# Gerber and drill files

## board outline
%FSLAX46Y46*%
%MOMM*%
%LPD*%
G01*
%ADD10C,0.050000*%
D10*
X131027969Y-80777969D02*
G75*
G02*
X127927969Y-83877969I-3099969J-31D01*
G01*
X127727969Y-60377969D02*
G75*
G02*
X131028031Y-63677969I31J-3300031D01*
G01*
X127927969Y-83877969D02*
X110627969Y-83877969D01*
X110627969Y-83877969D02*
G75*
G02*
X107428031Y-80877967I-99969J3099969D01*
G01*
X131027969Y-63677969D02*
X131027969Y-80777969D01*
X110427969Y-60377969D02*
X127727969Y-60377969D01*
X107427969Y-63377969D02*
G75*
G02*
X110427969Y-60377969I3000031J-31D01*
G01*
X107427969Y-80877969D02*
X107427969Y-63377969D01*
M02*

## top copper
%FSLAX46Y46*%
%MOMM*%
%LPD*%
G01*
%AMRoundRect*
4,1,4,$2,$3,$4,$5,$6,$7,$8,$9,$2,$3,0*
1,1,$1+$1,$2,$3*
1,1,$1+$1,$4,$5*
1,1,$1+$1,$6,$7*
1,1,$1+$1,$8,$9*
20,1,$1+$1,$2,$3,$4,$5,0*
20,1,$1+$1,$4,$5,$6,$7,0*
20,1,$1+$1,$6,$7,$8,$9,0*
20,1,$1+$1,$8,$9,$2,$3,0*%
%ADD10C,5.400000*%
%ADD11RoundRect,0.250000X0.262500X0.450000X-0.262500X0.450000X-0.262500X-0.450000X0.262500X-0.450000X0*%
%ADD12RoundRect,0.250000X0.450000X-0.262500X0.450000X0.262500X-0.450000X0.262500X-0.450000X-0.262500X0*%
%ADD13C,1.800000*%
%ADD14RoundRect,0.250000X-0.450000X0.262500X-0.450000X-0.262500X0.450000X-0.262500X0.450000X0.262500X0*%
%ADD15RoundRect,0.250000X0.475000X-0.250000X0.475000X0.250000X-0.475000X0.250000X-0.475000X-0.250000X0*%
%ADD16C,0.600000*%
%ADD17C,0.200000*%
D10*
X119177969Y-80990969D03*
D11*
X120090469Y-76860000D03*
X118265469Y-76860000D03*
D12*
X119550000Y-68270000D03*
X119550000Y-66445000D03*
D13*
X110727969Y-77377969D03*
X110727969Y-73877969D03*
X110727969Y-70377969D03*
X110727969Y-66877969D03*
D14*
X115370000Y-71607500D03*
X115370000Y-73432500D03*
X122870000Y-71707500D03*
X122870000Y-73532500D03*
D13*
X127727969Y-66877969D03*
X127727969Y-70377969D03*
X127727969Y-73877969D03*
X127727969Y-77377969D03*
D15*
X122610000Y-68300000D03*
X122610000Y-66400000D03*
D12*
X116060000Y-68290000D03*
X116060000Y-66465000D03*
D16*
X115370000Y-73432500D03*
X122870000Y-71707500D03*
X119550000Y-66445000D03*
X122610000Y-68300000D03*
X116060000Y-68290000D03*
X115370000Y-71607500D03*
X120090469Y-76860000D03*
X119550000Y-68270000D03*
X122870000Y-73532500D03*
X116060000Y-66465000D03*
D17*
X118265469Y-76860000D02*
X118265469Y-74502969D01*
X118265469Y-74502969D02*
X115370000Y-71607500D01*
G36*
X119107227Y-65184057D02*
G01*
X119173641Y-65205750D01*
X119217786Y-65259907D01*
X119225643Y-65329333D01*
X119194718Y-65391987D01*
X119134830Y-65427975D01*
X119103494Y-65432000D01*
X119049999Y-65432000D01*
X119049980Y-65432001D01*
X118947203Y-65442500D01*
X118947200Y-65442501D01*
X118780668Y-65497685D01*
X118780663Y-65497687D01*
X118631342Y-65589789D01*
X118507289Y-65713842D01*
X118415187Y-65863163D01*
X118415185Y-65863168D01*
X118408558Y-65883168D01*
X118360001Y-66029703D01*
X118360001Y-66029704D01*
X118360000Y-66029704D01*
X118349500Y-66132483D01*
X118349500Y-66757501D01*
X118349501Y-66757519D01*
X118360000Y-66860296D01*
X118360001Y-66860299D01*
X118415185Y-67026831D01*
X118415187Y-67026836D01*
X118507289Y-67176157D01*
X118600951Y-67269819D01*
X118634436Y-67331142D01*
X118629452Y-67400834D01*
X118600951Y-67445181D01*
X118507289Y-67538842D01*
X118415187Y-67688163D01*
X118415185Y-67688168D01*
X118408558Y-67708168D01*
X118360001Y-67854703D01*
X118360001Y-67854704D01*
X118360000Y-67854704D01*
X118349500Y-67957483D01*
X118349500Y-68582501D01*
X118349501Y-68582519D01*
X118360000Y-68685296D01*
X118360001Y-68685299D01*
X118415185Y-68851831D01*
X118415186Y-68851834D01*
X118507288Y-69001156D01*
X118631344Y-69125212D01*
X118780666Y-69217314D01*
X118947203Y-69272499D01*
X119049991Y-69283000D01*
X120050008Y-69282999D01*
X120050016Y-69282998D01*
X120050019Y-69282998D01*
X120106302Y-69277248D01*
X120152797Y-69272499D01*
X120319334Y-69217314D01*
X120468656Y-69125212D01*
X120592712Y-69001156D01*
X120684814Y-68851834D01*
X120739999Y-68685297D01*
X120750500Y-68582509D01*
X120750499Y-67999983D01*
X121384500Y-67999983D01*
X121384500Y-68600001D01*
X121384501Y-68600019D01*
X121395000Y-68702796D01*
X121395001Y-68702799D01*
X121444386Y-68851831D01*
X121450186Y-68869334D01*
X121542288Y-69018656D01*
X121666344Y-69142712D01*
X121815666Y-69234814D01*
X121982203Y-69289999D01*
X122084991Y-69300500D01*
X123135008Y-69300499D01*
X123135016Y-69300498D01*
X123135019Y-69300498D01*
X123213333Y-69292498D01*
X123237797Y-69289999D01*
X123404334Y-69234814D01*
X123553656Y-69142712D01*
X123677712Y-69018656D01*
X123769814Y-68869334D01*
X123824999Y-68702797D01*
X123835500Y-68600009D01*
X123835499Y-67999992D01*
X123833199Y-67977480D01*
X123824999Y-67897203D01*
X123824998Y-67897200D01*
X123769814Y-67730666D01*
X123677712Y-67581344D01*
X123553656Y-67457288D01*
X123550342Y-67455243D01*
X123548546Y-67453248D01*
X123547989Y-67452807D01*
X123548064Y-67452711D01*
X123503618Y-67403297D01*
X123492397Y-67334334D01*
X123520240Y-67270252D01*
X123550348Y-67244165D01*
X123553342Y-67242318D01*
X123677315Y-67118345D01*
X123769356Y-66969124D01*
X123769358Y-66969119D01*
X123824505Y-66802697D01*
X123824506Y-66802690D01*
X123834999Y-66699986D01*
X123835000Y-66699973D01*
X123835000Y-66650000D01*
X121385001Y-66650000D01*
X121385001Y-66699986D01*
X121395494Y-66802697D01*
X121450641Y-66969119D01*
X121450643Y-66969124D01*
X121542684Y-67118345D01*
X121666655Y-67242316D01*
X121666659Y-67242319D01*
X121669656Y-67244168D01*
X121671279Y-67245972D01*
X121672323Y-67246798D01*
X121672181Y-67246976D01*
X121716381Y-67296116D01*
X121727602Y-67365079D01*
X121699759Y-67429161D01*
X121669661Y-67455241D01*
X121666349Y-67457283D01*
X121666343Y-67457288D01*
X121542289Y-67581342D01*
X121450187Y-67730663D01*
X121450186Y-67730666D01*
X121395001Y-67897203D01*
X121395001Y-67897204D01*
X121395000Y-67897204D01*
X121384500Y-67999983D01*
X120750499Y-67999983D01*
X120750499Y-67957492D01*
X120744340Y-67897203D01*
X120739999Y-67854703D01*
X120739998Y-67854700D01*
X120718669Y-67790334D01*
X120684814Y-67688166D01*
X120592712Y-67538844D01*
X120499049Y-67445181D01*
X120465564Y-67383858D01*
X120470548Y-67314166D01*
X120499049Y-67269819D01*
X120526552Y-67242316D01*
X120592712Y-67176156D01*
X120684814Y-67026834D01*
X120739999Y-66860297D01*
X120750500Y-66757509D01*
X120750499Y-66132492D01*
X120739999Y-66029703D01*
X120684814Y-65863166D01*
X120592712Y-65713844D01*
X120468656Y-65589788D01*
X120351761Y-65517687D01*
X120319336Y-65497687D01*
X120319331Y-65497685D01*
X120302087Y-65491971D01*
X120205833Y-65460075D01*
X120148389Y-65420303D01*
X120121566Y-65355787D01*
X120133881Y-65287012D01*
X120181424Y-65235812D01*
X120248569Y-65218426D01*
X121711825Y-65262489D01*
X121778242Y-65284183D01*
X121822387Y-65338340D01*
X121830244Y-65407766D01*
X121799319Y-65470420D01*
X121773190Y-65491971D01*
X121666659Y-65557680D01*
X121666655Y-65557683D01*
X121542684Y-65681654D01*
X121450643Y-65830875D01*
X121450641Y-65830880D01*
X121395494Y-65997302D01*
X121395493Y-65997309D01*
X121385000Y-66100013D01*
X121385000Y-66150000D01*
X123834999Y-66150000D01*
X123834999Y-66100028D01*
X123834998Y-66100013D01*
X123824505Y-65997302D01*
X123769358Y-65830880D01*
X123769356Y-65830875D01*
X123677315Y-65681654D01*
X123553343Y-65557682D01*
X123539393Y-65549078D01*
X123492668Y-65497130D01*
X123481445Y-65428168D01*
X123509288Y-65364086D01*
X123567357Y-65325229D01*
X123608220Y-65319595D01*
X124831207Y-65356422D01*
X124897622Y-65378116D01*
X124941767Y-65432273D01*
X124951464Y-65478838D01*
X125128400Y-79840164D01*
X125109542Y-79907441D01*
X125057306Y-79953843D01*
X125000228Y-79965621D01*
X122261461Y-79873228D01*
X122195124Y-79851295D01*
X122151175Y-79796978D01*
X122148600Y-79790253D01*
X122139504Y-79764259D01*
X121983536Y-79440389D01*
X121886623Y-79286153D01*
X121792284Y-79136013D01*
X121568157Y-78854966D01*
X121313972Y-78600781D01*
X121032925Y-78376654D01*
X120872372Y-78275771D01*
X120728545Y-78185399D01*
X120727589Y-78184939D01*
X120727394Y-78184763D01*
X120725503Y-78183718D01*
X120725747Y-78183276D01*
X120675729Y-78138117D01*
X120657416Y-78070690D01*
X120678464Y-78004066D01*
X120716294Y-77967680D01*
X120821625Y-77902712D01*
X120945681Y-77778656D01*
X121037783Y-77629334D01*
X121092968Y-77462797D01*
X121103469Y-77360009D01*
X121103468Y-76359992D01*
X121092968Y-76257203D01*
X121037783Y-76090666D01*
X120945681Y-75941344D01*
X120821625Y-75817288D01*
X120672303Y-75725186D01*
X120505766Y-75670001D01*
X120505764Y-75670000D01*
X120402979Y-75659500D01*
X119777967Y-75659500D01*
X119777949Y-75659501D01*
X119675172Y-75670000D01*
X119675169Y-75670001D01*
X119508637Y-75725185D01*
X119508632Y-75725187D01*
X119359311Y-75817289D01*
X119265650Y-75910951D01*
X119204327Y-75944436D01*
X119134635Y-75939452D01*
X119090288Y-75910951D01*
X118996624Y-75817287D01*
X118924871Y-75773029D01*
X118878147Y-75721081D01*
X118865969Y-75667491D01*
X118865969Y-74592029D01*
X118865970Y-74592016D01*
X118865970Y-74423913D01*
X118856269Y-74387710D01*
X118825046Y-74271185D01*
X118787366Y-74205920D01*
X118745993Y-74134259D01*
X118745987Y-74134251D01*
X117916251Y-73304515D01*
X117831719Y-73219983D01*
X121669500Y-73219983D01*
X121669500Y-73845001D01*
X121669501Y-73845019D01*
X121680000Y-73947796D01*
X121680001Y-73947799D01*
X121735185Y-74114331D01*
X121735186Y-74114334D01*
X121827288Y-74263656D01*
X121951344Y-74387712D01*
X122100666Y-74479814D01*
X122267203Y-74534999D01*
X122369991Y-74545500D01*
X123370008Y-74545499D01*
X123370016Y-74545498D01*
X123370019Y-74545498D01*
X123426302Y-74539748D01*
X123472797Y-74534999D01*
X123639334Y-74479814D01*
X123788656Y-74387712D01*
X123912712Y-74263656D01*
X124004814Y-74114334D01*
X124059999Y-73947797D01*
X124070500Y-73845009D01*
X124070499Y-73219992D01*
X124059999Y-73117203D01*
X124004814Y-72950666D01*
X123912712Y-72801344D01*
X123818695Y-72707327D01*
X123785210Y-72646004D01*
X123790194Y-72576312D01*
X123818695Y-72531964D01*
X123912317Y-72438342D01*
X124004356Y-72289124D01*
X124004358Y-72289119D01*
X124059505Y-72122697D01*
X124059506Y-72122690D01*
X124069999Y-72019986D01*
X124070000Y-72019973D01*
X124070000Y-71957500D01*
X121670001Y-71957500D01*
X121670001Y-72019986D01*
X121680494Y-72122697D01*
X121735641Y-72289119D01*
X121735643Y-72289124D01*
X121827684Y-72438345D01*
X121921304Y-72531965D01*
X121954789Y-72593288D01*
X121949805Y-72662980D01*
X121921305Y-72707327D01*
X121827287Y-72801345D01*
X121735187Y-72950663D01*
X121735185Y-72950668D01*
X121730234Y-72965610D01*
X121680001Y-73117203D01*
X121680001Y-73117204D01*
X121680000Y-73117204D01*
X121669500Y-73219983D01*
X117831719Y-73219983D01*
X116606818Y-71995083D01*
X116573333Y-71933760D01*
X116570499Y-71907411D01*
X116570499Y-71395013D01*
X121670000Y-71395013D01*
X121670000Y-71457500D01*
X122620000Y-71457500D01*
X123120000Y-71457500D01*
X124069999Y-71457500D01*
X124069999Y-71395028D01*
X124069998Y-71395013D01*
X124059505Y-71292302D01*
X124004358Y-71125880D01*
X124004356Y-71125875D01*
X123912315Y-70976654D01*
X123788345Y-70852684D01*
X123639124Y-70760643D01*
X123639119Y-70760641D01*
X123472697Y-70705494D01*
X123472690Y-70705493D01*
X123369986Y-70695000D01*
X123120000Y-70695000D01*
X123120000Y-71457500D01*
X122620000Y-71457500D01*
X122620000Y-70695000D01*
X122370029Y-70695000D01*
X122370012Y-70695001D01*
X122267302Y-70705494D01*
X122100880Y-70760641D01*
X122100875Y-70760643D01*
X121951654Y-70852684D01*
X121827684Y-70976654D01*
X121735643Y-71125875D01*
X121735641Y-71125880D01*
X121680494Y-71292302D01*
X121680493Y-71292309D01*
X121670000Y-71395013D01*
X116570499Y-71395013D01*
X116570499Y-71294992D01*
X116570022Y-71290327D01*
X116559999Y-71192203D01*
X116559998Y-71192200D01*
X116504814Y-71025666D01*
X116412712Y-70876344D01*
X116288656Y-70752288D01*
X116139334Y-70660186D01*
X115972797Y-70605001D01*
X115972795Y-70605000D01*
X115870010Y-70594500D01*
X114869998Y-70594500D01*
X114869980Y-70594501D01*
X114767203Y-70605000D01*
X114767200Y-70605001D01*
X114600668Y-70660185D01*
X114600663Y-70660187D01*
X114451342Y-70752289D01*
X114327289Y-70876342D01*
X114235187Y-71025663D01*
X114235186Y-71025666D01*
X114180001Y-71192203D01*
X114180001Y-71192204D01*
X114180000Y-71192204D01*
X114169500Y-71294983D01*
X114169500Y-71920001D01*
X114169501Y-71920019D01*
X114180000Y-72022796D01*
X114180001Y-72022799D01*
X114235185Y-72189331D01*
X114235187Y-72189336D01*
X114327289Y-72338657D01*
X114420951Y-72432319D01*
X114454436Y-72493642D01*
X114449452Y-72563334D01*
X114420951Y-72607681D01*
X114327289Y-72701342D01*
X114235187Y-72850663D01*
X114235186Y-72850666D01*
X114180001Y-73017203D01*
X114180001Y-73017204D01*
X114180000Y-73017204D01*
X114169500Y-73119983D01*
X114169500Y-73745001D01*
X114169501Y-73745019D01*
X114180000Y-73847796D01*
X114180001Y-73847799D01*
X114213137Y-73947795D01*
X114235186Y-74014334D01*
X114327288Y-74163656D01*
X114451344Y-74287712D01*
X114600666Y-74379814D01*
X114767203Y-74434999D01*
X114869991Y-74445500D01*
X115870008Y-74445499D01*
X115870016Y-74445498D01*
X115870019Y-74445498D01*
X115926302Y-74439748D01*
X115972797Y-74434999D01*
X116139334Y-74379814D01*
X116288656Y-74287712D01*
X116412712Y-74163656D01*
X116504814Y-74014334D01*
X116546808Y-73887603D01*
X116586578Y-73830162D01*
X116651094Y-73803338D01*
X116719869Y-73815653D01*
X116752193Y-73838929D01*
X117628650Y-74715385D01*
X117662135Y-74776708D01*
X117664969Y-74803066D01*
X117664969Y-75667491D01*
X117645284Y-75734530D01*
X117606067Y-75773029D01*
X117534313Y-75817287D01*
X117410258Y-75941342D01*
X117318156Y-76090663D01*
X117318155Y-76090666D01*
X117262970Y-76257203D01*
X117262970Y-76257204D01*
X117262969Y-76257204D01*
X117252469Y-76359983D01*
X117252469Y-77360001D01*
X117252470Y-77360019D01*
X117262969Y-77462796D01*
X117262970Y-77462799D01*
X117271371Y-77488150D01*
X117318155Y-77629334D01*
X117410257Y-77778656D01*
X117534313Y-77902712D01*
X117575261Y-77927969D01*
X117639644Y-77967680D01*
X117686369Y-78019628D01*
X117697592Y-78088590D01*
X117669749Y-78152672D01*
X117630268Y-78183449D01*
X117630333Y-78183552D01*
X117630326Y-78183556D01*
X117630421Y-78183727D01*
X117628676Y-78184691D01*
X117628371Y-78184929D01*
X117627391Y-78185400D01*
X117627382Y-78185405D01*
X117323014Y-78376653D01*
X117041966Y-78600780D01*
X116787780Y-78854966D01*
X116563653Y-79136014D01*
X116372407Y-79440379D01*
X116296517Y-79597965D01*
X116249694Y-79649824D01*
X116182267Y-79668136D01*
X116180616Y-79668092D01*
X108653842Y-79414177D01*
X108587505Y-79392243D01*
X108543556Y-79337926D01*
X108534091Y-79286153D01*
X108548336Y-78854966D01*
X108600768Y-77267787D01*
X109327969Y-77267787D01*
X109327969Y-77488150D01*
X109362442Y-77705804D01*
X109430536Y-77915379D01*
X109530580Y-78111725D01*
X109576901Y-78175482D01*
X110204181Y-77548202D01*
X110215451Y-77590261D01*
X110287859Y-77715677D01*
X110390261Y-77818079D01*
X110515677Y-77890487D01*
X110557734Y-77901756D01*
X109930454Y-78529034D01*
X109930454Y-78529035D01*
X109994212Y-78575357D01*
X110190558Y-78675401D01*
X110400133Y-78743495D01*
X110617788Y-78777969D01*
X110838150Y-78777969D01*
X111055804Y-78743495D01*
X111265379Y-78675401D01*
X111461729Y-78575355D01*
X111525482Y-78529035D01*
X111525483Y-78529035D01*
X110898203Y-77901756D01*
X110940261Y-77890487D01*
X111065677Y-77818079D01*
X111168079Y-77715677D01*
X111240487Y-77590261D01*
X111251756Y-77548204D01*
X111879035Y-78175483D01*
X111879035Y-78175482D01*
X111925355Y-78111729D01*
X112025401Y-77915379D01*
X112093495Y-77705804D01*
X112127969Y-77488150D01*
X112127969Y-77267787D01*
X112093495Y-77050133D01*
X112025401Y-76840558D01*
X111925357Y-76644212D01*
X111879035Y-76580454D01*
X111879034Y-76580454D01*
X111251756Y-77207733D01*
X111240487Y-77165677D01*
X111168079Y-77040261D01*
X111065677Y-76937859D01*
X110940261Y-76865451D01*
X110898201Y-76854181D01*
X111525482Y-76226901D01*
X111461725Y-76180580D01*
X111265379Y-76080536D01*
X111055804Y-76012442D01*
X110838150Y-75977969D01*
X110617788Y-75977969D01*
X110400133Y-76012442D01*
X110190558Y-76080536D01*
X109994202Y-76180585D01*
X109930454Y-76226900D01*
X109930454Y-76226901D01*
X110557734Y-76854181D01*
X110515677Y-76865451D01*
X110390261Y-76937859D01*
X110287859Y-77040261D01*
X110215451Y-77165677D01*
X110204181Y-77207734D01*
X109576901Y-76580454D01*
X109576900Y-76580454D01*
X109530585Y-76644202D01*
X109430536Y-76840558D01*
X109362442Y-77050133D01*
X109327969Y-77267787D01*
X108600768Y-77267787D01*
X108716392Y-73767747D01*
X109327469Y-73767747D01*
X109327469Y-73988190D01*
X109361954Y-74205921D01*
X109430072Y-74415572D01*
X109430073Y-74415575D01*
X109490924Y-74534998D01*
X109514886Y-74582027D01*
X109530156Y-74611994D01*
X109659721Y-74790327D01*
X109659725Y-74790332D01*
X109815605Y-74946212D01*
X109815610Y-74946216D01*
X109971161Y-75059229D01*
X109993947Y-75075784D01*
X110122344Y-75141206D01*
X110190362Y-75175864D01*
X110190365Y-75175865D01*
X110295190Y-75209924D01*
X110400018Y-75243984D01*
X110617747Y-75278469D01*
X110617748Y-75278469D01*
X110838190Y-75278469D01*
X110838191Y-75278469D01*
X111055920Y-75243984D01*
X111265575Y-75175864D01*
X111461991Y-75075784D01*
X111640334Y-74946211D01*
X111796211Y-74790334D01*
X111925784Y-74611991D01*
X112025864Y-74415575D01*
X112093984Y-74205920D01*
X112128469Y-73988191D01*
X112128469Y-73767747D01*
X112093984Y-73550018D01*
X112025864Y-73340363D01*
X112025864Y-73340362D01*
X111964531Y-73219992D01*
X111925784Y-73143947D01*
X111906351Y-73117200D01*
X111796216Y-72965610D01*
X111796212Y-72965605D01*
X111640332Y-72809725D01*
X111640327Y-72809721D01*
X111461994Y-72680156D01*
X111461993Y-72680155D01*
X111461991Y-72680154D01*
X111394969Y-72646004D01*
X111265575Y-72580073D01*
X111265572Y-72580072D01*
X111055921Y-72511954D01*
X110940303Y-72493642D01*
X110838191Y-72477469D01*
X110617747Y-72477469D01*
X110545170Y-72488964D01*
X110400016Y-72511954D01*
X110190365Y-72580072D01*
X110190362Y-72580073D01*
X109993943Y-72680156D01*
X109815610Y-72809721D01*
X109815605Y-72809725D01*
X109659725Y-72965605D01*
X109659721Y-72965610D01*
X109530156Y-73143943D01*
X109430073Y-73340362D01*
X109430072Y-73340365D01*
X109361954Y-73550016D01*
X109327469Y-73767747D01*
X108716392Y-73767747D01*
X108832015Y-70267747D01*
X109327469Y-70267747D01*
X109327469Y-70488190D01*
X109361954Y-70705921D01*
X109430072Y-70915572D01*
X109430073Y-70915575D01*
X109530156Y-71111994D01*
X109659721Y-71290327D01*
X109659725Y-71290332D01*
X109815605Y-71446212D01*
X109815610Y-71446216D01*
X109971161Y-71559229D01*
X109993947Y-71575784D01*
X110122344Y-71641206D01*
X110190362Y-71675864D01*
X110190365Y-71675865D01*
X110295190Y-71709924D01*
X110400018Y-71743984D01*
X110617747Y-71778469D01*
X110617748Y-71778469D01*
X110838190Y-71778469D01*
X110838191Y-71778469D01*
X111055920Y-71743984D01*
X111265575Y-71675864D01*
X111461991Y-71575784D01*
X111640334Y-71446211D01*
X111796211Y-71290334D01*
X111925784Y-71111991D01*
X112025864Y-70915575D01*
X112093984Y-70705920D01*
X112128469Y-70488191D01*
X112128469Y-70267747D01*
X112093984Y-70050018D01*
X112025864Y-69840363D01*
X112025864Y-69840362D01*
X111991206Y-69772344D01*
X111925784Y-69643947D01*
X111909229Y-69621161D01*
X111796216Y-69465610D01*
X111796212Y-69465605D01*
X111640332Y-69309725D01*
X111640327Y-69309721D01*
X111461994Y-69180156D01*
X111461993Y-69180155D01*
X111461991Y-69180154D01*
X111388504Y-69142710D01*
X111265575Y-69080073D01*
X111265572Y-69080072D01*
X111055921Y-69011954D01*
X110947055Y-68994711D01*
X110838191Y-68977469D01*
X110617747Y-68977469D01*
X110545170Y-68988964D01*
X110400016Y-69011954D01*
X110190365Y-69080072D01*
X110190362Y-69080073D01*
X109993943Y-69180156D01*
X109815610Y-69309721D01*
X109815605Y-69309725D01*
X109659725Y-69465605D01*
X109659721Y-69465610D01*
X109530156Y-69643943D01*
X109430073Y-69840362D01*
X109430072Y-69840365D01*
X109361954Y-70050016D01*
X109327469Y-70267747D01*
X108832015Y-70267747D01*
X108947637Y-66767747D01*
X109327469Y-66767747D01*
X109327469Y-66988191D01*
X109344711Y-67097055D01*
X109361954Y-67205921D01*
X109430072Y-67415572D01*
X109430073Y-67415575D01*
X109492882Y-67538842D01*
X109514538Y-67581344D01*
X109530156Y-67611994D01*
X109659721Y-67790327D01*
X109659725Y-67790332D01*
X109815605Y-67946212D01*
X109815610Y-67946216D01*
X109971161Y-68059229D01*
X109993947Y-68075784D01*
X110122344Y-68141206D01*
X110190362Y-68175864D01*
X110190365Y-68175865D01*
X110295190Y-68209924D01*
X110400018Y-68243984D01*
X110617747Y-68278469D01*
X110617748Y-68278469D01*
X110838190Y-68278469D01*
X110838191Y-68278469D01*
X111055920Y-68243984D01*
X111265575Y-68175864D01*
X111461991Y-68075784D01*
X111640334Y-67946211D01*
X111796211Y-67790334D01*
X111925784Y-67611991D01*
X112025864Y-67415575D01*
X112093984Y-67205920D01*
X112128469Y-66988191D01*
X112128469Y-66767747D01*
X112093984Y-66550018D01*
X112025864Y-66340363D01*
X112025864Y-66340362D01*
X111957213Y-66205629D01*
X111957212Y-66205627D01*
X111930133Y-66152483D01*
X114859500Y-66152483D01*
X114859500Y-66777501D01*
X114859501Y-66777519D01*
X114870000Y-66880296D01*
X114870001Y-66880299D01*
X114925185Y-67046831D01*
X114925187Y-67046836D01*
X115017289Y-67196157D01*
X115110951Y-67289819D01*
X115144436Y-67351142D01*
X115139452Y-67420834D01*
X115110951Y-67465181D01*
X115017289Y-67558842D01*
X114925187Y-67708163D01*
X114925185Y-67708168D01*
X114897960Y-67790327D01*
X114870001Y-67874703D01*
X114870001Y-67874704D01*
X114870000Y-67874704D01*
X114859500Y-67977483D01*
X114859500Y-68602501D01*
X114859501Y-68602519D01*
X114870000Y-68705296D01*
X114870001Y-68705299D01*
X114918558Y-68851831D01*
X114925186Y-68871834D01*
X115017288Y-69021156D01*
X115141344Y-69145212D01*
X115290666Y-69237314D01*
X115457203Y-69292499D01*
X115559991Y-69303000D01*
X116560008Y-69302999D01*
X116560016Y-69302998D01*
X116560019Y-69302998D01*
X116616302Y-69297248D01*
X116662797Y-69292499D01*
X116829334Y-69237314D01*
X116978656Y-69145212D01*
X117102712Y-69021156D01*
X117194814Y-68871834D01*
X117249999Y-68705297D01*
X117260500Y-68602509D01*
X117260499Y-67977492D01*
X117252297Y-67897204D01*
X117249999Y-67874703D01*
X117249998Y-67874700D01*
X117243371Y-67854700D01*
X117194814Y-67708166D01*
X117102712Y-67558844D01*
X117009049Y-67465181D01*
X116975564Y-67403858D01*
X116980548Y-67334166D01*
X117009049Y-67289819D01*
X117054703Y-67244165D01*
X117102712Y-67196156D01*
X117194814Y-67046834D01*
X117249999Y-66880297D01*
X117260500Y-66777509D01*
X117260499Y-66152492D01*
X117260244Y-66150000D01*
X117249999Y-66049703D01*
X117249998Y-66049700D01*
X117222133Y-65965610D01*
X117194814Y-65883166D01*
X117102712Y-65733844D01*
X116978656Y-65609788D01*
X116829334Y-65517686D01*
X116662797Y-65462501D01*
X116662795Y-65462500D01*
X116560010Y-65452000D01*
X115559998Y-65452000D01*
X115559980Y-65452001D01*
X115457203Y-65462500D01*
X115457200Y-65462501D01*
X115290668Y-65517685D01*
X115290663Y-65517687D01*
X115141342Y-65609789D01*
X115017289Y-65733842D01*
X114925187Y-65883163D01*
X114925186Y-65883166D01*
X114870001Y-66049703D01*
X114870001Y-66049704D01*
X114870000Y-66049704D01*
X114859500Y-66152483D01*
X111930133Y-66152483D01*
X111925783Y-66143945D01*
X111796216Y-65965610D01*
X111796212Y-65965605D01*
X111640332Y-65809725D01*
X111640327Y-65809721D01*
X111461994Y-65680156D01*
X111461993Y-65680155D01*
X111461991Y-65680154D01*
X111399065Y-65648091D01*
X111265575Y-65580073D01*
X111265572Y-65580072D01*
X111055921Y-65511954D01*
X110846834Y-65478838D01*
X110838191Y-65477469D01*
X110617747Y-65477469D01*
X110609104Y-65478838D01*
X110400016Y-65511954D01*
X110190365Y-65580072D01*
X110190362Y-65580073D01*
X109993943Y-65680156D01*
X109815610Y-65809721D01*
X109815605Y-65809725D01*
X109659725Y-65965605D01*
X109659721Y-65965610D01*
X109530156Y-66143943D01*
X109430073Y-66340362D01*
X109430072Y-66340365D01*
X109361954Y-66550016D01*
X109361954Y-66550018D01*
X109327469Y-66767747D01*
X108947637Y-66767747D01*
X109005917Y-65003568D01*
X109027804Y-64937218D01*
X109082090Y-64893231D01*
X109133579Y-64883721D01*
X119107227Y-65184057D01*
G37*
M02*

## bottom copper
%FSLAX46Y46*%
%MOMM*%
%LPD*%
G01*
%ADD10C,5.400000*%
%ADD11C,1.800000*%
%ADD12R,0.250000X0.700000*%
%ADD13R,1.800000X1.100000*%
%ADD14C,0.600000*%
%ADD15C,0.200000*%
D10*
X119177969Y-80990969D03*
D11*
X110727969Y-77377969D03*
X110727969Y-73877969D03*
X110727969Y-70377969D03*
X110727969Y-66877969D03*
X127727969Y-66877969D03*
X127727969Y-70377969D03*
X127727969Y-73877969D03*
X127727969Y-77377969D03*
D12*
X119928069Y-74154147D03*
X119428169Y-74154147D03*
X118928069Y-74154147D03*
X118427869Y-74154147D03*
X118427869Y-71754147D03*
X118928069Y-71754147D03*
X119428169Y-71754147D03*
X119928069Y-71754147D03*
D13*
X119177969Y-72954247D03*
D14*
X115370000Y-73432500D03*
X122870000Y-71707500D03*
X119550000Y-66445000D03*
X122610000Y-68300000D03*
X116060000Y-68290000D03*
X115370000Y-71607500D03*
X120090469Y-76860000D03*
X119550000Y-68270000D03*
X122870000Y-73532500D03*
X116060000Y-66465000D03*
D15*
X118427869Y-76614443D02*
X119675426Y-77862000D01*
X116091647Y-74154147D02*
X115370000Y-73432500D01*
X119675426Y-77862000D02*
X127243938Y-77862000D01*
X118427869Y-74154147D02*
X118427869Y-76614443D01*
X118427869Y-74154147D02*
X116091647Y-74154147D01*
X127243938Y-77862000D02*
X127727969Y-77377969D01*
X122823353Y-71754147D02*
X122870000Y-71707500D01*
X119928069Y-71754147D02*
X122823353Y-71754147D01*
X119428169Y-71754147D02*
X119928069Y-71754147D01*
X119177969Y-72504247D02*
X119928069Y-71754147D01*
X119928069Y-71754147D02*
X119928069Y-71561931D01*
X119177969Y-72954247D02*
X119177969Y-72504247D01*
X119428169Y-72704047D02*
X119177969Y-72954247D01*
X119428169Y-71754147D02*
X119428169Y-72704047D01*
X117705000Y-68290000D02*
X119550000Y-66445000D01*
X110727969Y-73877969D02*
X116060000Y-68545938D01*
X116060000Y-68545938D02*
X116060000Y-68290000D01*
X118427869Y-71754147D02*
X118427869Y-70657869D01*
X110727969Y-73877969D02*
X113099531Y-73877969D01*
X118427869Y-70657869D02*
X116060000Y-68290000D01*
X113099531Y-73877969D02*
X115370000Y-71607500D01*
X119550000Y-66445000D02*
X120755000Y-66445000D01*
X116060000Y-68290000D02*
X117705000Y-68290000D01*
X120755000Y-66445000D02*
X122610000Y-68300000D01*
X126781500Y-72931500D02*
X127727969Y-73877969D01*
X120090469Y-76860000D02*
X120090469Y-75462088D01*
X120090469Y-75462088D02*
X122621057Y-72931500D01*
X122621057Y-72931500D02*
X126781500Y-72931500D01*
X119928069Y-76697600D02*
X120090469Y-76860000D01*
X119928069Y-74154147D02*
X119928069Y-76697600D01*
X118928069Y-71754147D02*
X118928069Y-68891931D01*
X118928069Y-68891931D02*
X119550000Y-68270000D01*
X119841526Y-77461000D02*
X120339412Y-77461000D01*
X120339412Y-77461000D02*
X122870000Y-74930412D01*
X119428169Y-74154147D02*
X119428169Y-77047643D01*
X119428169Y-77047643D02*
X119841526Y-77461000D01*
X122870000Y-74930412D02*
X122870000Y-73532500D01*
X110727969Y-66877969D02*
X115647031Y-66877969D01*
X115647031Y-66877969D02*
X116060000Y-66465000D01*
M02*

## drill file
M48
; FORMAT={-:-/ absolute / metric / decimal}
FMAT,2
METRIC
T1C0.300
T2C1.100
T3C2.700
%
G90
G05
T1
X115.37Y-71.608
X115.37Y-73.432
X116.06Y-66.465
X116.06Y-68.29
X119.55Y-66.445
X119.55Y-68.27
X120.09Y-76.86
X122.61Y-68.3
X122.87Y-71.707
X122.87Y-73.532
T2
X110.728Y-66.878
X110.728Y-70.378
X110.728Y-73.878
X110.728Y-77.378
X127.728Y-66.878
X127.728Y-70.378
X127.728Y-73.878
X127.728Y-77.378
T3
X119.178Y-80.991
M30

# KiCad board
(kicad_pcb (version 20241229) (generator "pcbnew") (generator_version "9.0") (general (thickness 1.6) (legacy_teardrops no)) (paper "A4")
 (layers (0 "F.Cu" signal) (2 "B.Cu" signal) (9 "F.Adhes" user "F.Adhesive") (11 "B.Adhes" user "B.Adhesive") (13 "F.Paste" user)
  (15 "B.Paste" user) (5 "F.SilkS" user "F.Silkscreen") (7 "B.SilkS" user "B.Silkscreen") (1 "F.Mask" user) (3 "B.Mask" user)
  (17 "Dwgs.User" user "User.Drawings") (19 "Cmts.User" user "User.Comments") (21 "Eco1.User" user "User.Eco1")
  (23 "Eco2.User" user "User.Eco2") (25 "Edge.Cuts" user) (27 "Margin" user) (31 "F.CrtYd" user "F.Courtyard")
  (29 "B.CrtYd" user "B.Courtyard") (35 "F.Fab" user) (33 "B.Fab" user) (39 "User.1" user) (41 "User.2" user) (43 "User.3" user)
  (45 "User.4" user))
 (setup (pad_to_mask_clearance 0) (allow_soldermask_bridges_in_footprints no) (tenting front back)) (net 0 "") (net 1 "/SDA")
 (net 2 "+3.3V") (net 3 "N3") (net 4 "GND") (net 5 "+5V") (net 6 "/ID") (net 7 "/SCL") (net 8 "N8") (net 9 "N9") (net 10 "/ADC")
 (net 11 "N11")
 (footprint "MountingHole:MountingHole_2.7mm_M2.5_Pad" (layer "F.Cu") (at 119.177969 80.990969)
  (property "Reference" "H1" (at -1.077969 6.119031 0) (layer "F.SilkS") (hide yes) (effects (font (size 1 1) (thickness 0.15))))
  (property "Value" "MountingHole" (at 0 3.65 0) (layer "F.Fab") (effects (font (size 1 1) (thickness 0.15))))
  (pad "1" thru_hole circle (at 0 0) (size 5.4 5.4) (drill 2.7) (layers "*.Cu" "*.Mask") (remove_unused_layers no) (zone_connect 2)))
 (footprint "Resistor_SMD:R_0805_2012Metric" (layer "F.Cu") (at 119.177969 76.86 180)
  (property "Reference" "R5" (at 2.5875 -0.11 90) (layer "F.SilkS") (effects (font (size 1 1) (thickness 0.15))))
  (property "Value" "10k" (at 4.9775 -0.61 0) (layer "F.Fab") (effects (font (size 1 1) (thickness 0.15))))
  (pad "1" smd roundrect (at -0.9125 0 180) (size 1.025 1.4) (layers "F.Cu" "F.Mask" "F.Paste") (roundrect_rratio 0.243902) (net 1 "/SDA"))
  (pad "2" smd roundrect (at 0.9125 0 180) (size 1.025 1.4) (layers "F.Cu" "F.Mask" "F.Paste") (roundrect_rratio 0.243902) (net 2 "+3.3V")))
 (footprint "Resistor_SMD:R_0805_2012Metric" (layer "F.Cu") (at 119.55 67.3575 90)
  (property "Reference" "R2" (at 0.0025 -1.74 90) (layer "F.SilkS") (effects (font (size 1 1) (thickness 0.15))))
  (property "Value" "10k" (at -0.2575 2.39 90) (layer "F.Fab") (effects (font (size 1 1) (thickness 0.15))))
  (pad "1" smd roundrect (at -0.9125 0 90) (size 1.025 1.4) (layers "F.Cu" "F.Mask" "F.Paste") (roundrect_rratio 0.243902) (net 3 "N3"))
  (pad "2" smd roundrect (at 0.9125 0 90) (size 1.025 1.4) (layers "F.Cu" "F.Mask" "F.Paste") (roundrect_rratio 0.243902) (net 2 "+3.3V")))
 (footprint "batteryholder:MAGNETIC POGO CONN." (layer "F.Cu") (at 110.727969 72.127969 90)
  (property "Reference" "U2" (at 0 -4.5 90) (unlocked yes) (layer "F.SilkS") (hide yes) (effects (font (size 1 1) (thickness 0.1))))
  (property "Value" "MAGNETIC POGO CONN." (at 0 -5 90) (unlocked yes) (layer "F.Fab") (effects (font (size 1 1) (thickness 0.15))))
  (pad "1" thru_hole circle (at -5.25 0 90) (size 1.8 1.8) (drill 1.1) (layers "*.Cu" "*.Mask") (remove_unused_layers no) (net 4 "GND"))
  (pad "2" thru_hole circle (at -1.75 0 90) (size 1.8 1.8) (drill 1.1) (layers "*.Cu" "*.Mask") (remove_unused_layers no) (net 2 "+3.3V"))
  (pad "3" thru_hole circle (at 1.75 0 90) (size 1.8 1.8) (drill 1.1) (layers "*.Cu" "*.Mask") (remove_unused_layers no) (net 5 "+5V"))
  (pad "4" thru_hole circle (at 5.25 0 90) (size 1.8 1.8) (drill 1.1) (layers "*.Cu" "*.Mask") (remove_unused_layers no) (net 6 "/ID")))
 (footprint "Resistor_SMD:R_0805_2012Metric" (layer "F.Cu") (at 115.37 72.52 -90)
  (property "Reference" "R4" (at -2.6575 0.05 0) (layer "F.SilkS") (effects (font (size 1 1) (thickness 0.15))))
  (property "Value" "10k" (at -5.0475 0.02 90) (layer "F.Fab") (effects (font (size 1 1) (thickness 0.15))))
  (pad "1" smd roundrect (at -0.9125 0 270) (size 1.025 1.4) (layers "F.Cu" "F.Mask" "F.Paste") (roundrect_rratio 0.243902) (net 2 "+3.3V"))
  (pad "2" smd roundrect (at 0.9125 0 270) (size 1.025 1.4) (layers "F.Cu" "F.Mask" "F.Paste") (roundrect_rratio 0.243902) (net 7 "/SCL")))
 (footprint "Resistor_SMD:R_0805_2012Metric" (layer "F.Cu") (at 122.87 72.62 -90)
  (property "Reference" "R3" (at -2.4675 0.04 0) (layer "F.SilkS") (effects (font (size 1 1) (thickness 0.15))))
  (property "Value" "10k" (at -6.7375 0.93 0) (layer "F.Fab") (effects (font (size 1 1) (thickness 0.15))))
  (pad "1" smd roundrect (at -0.9125 0 270) (size 1.025 1.4) (layers "F.Cu" "F.Mask" "F.Paste") (roundrect_rratio 0.243902) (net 4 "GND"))
  (pad "2" smd roundrect (at 0.9125 0 270) (size 1.025 1.4) (layers "F.Cu" "F.Mask" "F.Paste") (roundrect_rratio 0.243902) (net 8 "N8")))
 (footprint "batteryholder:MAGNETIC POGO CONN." (layer "F.Cu") (at 127.727969 72.127969 -90)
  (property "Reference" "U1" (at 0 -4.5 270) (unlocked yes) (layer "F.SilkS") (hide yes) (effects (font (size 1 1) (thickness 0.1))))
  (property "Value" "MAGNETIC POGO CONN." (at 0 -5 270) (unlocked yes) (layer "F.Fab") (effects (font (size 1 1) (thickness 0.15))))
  (pad "1" thru_hole circle (at -5.25 0 270) (size 1.8 1.8) (drill 1.1) (layers "*.Cu" "*.Mask") (remove_unused_layers no) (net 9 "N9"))
  (pad "2" thru_hole circle (at -1.75 0 270) (size 1.8 1.8) (drill 1.1) (layers "*.Cu" "*.Mask") (remove_unused_layers no) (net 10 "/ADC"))
  (pad "3" thru_hole circle (at 1.75 0 270) (size 1.8 1.8) (drill 1.1) (layers "*.Cu" "*.Mask") (remove_unused_layers no) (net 1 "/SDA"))
  (pad "4" thru_hole circle (at 5.25 0 270) (size 1.8 1.8) (drill 1.1) (layers "*.Cu" "*.Mask") (remove_unused_layers no) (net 7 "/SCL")))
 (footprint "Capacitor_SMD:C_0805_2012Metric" (layer "F.Cu") (at 122.61 67.35 90)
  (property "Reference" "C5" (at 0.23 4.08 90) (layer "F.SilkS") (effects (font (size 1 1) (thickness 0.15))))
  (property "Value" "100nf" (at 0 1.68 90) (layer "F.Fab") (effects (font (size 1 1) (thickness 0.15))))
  (pad "1" smd roundrect (at -0.95 0 90) (size 1 1.45) (layers "F.Cu" "F.Mask" "F.Paste") (roundrect_rratio 0.25) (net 2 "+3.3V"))
  (pad "2" smd roundrect (at 0.95 0 90) (size 1 1.45) (layers "F.Cu" "F.Mask" "F.Paste") (roundrect_rratio 0.25) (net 4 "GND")))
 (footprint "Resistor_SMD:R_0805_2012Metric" (layer "F.Cu") (at 116.06 67.3775 90)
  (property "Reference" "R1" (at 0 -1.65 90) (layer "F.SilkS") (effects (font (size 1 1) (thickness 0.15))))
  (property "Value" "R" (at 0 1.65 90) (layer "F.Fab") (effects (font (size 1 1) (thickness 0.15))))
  (pad "1" smd roundrect (at -0.9125 0 90) (size 1.025 1.4) (layers "F.Cu" "F.Mask" "F.Paste") (roundrect_rratio 0.243902) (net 2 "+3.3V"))
  (pad "2" smd roundrect (at 0.9125 0 90) (size 1.025 1.4) (layers "F.Cu" "F.Mask" "F.Paste") (roundrect_rratio 0.243902) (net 6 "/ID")))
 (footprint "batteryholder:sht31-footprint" (layer "B.Cu") (at 119.177969 72.954147 180)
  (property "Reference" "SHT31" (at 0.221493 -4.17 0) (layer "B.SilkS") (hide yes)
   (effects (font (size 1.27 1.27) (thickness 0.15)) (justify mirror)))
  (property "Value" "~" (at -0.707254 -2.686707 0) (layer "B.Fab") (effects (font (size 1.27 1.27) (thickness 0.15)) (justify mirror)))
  (pad "1" smd rect (at -0.7501 -1.2 180) (size 0.25 0.7) (layers "B.Cu" "B.Mask" "B.Paste") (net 1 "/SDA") (solder_mask_margin 0.0508)
   (solder_paste_margin 0) (thermal_bridge_angle 0))
  (pad "2" smd rect (at -0.2502 -1.2 180) (size 0.25 0.7) (layers "B.Cu" "B.Mask" "B.Paste") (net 8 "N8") (solder_mask_margin 0.0508)
   (solder_paste_margin 0) (thermal_bridge_angle 0))
  (pad "3" smd rect (at 0.2499 -1.2 180) (size 0.25 0.7) (layers "B.Cu" "B.Mask" "B.Paste") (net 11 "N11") (solder_mask_margin 0.0508)
   (solder_paste_margin 0) (thermal_bridge_angle 0))
  (pad "4" smd rect (at 0.7501 -1.2 180) (size 0.25 0.7) (layers "B.Cu" "B.Mask" "B.Paste") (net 7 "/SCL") (solder_mask_margin 0.0508)
   (solder_paste_margin 0) (thermal_bridge_angle 0))
  (pad "5" smd rect (at 0.7501 1.2 180) (size 0.25 0.7) (layers "B.Cu" "B.Mask" "B.Paste") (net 2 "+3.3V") (solder_mask_margin 0.0508)
   (solder_paste_margin 0) (thermal_bridge_angle 0))
  (pad "6" smd rect (at 0.2499 1.2 180) (size 0.25 0.7) (layers "B.Cu" "B.Mask" "B.Paste") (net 3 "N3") (solder_mask_margin 0.0508)
   (solder_paste_margin 0) (thermal_bridge_angle 0))
  (pad "7" smd rect (at -0.2502 1.2 180) (size 0.25 0.7) (layers "B.Cu" "B.Mask" "B.Paste") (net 4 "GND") (solder_mask_margin 0.0508)
   (solder_paste_margin 0) (thermal_bridge_angle 0))
  (pad "8" smd rect (at -0.7501 1.2 180) (size 0.25 0.7) (layers "B.Cu" "B.Mask" "B.Paste") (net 4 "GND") (solder_mask_margin 0.0508)
   (solder_paste_margin 0) (thermal_bridge_angle 0))
  (pad "9" smd rect (at 0 -0.0001 180) (size 1.8 1.1) (layers "B.Cu" "B.Mask" "B.Paste") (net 4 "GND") (solder_mask_margin 0.0508)
   (solder_paste_margin 0) (thermal_bridge_angle 0))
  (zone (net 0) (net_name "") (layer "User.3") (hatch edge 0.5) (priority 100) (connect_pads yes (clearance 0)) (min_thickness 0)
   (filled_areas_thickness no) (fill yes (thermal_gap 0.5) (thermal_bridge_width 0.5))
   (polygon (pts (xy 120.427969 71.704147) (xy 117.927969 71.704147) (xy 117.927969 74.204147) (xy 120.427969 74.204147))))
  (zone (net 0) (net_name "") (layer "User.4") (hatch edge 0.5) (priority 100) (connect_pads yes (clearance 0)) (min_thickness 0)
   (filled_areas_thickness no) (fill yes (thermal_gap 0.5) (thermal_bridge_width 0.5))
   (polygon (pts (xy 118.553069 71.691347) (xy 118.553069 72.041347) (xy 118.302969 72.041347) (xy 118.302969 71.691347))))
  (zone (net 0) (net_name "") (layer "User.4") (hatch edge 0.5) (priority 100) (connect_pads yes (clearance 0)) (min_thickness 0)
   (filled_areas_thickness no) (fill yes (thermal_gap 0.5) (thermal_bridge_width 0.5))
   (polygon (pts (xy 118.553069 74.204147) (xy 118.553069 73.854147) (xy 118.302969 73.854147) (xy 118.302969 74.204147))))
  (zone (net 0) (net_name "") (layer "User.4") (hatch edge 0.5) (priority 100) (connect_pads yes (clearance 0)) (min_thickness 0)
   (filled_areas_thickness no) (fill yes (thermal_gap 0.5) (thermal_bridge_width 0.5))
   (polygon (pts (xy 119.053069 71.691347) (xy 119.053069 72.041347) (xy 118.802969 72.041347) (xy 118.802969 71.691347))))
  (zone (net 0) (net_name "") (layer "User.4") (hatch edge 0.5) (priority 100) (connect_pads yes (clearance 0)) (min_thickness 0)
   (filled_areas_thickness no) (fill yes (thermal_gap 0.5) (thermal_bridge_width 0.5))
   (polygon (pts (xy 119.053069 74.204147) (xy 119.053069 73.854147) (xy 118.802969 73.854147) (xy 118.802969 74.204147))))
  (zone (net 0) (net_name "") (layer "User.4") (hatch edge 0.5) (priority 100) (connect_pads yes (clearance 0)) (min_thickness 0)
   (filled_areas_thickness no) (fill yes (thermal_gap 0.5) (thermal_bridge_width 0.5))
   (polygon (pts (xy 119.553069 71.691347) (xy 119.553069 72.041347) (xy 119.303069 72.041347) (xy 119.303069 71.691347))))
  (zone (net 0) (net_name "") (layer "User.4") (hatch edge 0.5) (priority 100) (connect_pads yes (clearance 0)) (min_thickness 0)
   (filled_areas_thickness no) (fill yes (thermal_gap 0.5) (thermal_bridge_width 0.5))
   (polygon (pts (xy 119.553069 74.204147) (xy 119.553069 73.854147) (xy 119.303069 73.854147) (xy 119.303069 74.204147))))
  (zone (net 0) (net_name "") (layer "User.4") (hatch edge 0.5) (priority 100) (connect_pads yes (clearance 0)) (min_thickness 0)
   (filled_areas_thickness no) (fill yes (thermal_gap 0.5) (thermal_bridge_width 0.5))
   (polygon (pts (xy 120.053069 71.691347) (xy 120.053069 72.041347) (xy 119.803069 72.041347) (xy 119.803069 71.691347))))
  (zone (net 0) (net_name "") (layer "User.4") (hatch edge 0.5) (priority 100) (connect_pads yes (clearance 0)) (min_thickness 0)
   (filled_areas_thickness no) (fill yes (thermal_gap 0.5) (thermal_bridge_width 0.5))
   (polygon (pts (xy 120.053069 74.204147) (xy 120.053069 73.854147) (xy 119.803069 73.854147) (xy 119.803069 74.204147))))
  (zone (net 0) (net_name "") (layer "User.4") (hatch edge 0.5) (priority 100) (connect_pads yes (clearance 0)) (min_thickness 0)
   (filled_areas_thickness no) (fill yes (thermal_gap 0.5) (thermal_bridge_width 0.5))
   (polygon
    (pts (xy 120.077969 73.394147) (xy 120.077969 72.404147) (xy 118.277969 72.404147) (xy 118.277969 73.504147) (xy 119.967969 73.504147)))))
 (gr_arc (start 131.027969 80.777969) (mid 130.12 82.97) (end 127.927969 83.877969) (stroke (width 0.05) (type default)) (layer "Edge.Cuts"))
 (gr_arc (start 127.727969 60.377969) (mid 130.061421 61.344517) (end 131.027969 63.677969) (stroke (width 0.05) (type default))
  (layer "Edge.Cuts"))
 (gr_line (start 127.927969 83.877969) (end 110.627969 83.877969) (stroke (width 0.05) (type solid)) (layer "Edge.Cuts"))
 (gr_arc (start 110.627969 83.877969) (mid 108.406649 83.040711) (end 107.427969 80.877969) (stroke (width 0.05) (type default))
  (layer "Edge.Cuts"))
 (gr_line (start 131.027969 63.677969) (end 131.027969 80.777969) (stroke (width 0.05) (type default)) (layer "Edge.Cuts"))
 (gr_line (start 110.427969 60.377969) (end 127.727969 60.377969) (stroke (width 0.05) (type default)) (layer "Edge.Cuts"))
 (gr_arc (start 107.427969 63.377969) (mid 108.306649 61.256649) (end 110.427969 60.377969) (stroke (width 0.05) (type default))
  (layer "Edge.Cuts"))
 (gr_line (start 107.427969 80.877969) (end 107.427969 63.377969) (stroke (width 0.05) (type default)) (layer "Edge.Cuts"))
 (via blind (at 115.37 73.4325) (size 0.6) (drill 0.3) (layers "F.Cu" "B.Cu") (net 7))
 (segment (start 118.427869 76.614443) (end 119.675426 77.862) (width 0.2) (layer "B.Cu") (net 7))
 (segment (start 116.091647 74.154147) (end 115.37 73.4325) (width 0.2) (layer "B.Cu") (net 7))
 (segment (start 119.675426 77.862) (end 127.243938 77.862) (width 0.2) (layer "B.Cu") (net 7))
 (segment (start 118.427869 74.154147) (end 118.427869 76.614443) (width 0.2) (layer "B.Cu") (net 7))
 (segment (start 118.427869 74.154147) (end 116.091647 74.154147) (width 0.2) (layer "B.Cu") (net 7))
 (segment (start 127.243938 77.862) (end 127.727969 77.377969) (width 0.2) (layer "B.Cu") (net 7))
 (via blind (at 122.87 71.7075) (size 0.6) (drill 0.3) (layers "F.Cu" "B.Cu") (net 4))
 (segment (start 122.823353 71.754147) (end 122.87 71.7075) (width 0.2) (layer "B.Cu") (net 4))
 (segment (start 119.928069 71.754147) (end 122.823353 71.754147) (width 0.2) (layer "B.Cu") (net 4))
 (segment (start 119.428169 71.754147) (end 119.928069 71.754147) (width 0.2) (layer "B.Cu") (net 4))
 (segment (start 119.177969 72.504247) (end 119.928069 71.754147) (width 0.2) (layer "B.Cu") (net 4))
 (segment (start 119.928069 71.754147) (end 119.928069 71.561931) (width 0.2) (layer "B.Cu") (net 4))
 (segment (start 119.177969 72.954247) (end 119.177969 72.504247) (width 0.2) (layer "B.Cu") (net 4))
 (segment (start 119.428169 72.704047) (end 119.177969 72.954247) (width 0.2) (layer "B.Cu") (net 4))
 (segment (start 119.428169 71.754147) (end 119.428169 72.704047) (width 0.2) (layer "B.Cu") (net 4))
 (segment (start 118.265469 76.86) (end 118.265469 74.502969) (width 0.2) (layer "F.Cu") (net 2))
 (segment (start 118.265469 74.502969) (end 115.37 71.6075) (width 0.2) (layer "F.Cu") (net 2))
 (via blind (at 119.55 66.445) (size 0.6) (drill 0.3) (layers "F.Cu" "B.Cu") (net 2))
 (via blind (at 122.61 68.3) (size 0.6) (drill 0.3) (layers "F.Cu" "B.Cu") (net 2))
 (via blind (at 116.06 68.29) (size 0.6) (drill 0.3) (layers "F.Cu" "B.Cu") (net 2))
 (via blind (at 115.37 71.6075) (size 0.6) (drill 0.3) (layers "F.Cu" "B.Cu") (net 2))
 (segment (start 117.705 68.29) (end 119.55 66.445) (width 0.2) (layer "B.Cu") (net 2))
 (segment (start 110.727969 73.877969) (end 116.06 68.545938) (width 0.2) (layer "B.Cu") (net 2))
 (segment (start 116.06 68.545938) (end 116.06 68.29) (width 0.2) (layer "B.Cu") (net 2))
 (segment (start 118.427869 71.754147) (end 118.427869 70.657869) (width 0.2) (layer "B.Cu") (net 2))
 (segment (start 110.727969 73.877969) (end 113.099531 73.877969) (width 0.2) (layer "B.Cu") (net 2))
 (segment (start 118.427869 70.657869) (end 116.06 68.29) (width 0.2) (layer "B.Cu") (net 2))
 (segment (start 113.099531 73.877969) (end 115.37 71.6075) (width 0.2) (layer "B.Cu") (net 2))
 (segment (start 119.55 66.445) (end 120.755 66.445) (width 0.2) (layer "B.Cu") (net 2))
 (segment (start 116.06 68.29) (end 117.705 68.29) (width 0.2) (layer "B.Cu") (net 2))
 (segment (start 120.755 66.445) (end 122.61 68.3) (width 0.2) (layer "B.Cu") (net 2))
 (via blind (at 120.090469 76.86) (size 0.6) (drill 0.3) (layers "F.Cu" "B.Cu") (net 1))
 (segment (start 126.7815 72.9315) (end 127.727969 73.877969) (width 0.2) (layer "B.Cu") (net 1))
 (segment (start 120.090469 76.86) (end 120.090469 75.462088) (width 0.2) (layer "B.Cu") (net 1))
 (segment (start 120.090469 75.462088) (end 122.621057 72.9315) (width 0.2) (layer "B.Cu") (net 1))
 (segment (start 122.621057 72.9315) (end 126.7815 72.9315) (width 0.2) (layer "B.Cu") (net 1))
 (segment (start 119.928069 76.6976) (end 120.090469 76.86) (width 0.2) (layer "B.Cu") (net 1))
 (segment (start 119.928069 74.154147) (end 119.928069 76.6976) (width 0.2) (layer "B.Cu") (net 1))
 (via blind (at 119.55 68.27) (size 0.6) (drill 0.3) (layers "F.Cu" "B.Cu") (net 3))
 (segment (start 118.928069 71.754147) (end 118.928069 68.891931) (width 0.2) (layer "B.Cu") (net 3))
 (segment (start 118.928069 68.891931) (end 119.55 68.27) (width 0.2) (layer "B.Cu") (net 3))
 (via blind (at 122.87 73.5325) (size 0.6) (drill 0.3) (layers "F.Cu" "B.Cu") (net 8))
 (segment (start 119.841526 77.461) (end 120.339412 77.461) (width 0.2) (layer "B.Cu") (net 8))
 (segment (start 120.339412 77.461) (end 122.87 74.930412) (width 0.2) (layer "B.Cu") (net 8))
 (segment (start 119.428169 74.154147) (end 119.428169 77.047643) (width 0.2) (layer "B.Cu") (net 8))
 (segment (start 119.428169 77.047643) (end 119.841526 77.461) (width 0.2) (layer "B.Cu") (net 8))
 (segment (start 122.87 74.930412) (end 122.87 73.5325) (width 0.2) (layer "B.Cu") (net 8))
 (via blind (at 116.06 66.465) (size 0.6) (drill 0.3) (layers "F.Cu" "B.Cu") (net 6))
 (segment (start 110.727969 66.877969) (end 115.647031 66.877969) (width 0.2) (layer "B.Cu") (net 6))
 (segment (start 115.647031 66.877969) (end 116.06 66.465) (width 0.2) (layer "B.Cu") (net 6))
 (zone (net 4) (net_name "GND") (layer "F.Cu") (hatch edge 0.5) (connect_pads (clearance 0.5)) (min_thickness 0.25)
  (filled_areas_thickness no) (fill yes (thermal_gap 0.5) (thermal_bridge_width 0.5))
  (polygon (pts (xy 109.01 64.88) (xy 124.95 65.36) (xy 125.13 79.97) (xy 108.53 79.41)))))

